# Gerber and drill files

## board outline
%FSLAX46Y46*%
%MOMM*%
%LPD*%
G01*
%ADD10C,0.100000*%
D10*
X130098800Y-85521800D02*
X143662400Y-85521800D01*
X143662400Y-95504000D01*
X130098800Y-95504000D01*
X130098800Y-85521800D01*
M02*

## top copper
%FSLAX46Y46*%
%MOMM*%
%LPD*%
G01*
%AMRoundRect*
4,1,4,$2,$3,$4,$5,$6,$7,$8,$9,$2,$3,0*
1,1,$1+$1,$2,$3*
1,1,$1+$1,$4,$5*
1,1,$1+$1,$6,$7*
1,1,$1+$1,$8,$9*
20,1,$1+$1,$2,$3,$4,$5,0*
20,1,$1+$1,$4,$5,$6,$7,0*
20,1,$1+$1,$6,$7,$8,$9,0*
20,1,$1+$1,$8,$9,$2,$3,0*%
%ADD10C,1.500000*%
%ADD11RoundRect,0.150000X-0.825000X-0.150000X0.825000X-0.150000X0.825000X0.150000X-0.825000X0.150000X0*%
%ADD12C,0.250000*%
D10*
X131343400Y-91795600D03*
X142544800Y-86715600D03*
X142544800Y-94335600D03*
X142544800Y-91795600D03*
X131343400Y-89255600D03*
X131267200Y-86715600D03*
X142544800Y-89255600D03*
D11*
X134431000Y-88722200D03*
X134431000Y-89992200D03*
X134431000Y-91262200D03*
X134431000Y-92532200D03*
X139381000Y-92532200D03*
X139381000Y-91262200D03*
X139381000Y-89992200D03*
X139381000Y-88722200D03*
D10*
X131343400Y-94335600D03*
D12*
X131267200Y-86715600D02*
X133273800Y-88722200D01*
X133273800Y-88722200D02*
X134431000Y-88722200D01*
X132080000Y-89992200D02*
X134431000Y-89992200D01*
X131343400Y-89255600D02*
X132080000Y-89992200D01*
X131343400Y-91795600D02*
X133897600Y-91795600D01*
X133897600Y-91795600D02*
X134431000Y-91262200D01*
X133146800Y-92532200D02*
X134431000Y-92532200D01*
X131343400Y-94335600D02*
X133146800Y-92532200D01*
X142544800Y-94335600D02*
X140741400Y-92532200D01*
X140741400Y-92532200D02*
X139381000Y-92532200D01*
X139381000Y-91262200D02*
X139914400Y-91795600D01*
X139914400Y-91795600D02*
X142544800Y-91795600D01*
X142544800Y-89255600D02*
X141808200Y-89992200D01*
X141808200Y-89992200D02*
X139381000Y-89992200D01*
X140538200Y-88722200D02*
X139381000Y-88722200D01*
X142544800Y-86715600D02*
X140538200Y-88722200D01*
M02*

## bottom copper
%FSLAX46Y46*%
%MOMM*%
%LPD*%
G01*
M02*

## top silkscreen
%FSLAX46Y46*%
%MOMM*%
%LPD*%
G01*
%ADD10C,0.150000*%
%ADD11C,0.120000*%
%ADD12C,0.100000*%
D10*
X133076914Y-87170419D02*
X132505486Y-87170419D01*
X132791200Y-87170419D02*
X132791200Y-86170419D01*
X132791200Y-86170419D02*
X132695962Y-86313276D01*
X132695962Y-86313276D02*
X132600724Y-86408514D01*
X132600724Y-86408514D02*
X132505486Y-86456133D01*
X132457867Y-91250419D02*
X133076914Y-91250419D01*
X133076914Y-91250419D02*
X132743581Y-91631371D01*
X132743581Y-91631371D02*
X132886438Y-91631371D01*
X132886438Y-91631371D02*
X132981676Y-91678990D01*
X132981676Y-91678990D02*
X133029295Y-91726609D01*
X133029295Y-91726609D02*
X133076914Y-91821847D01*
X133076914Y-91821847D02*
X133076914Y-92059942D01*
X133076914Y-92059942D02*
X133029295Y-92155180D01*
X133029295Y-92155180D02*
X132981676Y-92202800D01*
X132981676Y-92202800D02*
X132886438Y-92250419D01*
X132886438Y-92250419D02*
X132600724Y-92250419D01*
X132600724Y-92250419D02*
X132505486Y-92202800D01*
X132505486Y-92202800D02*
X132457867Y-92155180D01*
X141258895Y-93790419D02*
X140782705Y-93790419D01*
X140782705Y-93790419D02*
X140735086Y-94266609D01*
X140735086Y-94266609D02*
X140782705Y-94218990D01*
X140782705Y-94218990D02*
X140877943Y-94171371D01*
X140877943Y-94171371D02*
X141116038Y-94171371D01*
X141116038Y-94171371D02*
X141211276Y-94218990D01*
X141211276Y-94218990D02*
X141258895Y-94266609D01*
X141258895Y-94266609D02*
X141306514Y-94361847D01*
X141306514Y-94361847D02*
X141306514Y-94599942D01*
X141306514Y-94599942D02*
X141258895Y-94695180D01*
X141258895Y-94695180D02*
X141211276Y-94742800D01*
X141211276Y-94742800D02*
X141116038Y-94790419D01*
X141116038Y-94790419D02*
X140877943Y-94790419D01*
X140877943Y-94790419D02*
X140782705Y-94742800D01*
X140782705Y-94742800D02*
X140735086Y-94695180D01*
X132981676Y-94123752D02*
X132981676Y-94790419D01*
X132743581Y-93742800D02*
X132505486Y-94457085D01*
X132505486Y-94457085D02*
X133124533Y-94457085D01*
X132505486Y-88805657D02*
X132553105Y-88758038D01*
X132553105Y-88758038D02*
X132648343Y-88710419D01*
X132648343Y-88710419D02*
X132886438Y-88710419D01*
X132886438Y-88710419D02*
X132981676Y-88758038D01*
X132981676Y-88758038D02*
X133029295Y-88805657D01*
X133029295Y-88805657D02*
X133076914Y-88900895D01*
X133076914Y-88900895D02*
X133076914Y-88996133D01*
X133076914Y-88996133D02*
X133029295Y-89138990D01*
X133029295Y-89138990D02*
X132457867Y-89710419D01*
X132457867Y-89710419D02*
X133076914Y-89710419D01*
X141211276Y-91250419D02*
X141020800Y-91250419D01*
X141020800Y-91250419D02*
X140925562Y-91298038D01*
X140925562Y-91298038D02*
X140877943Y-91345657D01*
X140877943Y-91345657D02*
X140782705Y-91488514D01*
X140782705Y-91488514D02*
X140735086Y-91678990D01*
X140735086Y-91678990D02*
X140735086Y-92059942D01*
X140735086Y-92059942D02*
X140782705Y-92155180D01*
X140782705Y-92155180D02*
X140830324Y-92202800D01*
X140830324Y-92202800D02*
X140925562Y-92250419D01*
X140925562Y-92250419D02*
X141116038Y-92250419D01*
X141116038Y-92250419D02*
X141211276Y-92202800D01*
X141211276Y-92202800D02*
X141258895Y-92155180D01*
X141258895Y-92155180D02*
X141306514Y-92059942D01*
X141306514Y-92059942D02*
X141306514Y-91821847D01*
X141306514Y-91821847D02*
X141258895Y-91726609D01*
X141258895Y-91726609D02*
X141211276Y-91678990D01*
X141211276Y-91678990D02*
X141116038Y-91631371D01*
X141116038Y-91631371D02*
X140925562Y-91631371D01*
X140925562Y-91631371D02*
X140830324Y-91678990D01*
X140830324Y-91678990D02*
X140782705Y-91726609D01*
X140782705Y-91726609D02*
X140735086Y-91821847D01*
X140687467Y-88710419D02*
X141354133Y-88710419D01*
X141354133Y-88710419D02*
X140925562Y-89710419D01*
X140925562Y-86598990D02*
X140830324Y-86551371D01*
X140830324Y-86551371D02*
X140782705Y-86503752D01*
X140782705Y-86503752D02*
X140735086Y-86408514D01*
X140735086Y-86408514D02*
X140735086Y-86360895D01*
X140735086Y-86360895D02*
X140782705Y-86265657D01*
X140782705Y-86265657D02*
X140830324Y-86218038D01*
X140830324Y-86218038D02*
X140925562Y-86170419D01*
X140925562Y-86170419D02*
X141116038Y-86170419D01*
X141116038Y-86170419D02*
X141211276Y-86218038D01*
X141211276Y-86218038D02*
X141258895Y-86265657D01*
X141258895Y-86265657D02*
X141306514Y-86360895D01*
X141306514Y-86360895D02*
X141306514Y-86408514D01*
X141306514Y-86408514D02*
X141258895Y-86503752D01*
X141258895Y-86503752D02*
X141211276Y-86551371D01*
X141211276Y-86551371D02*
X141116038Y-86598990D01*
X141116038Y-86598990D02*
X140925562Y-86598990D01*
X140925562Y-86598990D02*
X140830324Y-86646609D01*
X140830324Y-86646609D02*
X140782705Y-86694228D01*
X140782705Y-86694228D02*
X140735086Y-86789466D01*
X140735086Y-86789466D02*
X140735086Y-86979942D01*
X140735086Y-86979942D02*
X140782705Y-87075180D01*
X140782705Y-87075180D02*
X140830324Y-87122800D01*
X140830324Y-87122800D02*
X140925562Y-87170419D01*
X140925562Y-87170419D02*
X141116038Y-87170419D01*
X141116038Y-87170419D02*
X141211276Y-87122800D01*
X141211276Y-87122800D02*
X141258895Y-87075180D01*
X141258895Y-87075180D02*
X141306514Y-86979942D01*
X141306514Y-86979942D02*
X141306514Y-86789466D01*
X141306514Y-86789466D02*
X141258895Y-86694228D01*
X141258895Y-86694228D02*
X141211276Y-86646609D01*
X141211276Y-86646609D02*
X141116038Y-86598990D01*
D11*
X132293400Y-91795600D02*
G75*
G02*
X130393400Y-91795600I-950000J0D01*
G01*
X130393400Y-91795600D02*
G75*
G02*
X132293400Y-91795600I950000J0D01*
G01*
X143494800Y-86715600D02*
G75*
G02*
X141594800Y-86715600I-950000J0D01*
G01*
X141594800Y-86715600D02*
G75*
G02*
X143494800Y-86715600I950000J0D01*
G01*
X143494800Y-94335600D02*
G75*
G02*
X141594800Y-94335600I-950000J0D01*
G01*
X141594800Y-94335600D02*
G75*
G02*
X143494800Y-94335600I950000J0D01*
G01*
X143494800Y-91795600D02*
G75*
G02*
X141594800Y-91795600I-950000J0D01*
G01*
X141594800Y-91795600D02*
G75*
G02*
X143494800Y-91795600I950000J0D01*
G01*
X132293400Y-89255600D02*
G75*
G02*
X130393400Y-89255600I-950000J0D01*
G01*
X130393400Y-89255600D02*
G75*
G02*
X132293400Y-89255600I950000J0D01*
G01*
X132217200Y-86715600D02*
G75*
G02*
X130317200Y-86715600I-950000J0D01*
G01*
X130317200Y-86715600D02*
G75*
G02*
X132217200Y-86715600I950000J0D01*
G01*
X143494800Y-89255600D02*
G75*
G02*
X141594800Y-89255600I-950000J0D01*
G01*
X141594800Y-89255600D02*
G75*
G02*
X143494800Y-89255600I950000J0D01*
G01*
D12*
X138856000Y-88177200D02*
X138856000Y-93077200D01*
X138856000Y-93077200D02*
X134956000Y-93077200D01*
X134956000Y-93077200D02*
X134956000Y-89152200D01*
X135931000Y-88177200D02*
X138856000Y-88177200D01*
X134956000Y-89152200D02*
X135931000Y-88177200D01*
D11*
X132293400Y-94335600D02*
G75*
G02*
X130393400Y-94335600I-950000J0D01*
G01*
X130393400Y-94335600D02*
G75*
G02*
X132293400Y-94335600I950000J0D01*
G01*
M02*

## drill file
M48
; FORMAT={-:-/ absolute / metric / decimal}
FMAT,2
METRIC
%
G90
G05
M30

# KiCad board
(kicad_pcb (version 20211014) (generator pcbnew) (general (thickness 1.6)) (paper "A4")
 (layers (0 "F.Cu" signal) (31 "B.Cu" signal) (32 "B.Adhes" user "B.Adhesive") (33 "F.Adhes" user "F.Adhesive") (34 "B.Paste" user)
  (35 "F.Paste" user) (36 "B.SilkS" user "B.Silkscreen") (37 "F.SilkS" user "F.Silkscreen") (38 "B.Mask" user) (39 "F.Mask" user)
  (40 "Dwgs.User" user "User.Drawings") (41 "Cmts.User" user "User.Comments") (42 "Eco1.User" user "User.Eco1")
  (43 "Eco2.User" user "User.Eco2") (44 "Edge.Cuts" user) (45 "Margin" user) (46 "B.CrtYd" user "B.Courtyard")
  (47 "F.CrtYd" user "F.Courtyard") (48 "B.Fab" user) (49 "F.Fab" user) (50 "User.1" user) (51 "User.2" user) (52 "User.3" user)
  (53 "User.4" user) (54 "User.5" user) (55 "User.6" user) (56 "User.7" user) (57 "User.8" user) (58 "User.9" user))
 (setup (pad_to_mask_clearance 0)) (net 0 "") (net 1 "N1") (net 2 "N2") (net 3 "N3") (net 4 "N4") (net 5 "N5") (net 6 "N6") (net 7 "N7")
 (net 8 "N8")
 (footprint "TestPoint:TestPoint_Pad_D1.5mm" (layer "F.Cu") (at 131.3434 91.7956)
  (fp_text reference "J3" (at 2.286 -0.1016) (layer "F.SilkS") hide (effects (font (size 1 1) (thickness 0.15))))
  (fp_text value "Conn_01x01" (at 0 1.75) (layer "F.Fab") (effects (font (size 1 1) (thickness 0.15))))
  (fp_circle (center 0 0) (end 0 0.95) (layer "F.SilkS") (width 0.12) (fill none))
  (pad "1" smd circle (at 0 0) (size 1.5 1.5) (layers "F.Cu" "F.Mask") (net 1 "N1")))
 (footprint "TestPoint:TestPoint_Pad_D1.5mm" (layer "F.Cu") (at 142.5448 86.7156)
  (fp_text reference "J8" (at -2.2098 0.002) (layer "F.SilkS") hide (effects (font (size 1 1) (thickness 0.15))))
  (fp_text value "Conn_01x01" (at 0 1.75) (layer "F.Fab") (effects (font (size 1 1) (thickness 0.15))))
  (fp_circle (center 0 0) (end 0 0.95) (layer "F.SilkS") (width 0.12) (fill none))
  (pad "1" smd circle (at 0 0) (size 1.5 1.5) (layers "F.Cu" "F.Mask") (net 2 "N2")))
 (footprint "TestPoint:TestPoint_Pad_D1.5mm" (layer "F.Cu") (at 142.5448 94.3356)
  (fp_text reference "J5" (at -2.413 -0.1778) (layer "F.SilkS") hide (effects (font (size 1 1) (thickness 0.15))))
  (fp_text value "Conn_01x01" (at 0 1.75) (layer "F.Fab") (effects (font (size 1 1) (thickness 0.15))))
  (fp_circle (center 0 0) (end 0 0.95) (layer "F.SilkS") (width 0.12) (fill none))
  (pad "1" smd circle (at 0 0) (size 1.5 1.5) (layers "F.Cu" "F.Mask") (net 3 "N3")))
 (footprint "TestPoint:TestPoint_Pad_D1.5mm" (layer "F.Cu") (at 142.5448 91.7956)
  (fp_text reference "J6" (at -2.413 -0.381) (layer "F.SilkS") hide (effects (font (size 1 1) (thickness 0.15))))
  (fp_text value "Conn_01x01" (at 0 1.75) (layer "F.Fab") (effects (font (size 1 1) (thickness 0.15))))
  (fp_circle (center 0 0) (end 0 0.95) (layer "F.SilkS") (width 0.12) (fill none))
  (pad "1" smd circle (at 0 0) (size 1.5 1.5) (layers "F.Cu" "F.Mask") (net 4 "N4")))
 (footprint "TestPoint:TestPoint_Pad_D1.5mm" (layer "F.Cu") (at 131.3434 89.2556)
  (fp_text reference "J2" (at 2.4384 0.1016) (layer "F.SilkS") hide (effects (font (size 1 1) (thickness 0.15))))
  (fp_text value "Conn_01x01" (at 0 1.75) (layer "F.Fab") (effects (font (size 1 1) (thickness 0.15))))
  (fp_circle (center 0 0) (end 0 0.95) (layer "F.SilkS") (width 0.12) (fill none))
  (pad "1" smd circle (at 0 0) (size 1.5 1.5) (layers "F.Cu" "F.Mask") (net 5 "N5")))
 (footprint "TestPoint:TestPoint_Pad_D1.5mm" (layer "F.Cu") (at 131.2672 86.7156)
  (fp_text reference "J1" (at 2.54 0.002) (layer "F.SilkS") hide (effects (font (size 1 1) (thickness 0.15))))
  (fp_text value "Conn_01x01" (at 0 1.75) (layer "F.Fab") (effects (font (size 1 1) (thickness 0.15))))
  (fp_circle (center 0 0) (end 0 0.95) (layer "F.SilkS") (width 0.12) (fill none))
  (pad "1" smd circle (at 0 0) (size 1.5 1.5) (layers "F.Cu" "F.Mask") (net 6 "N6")))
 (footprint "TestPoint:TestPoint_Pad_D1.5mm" (layer "F.Cu") (at 142.5448 89.2556)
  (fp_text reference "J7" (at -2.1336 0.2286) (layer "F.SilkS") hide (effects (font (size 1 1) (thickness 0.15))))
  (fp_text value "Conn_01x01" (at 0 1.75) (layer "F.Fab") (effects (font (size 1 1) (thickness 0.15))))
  (fp_circle (center 0 0) (end 0 0.95) (layer "F.SilkS") (width 0.12) (fill none))
  (pad "1" smd circle (at 0 0) (size 1.5 1.5) (layers "F.Cu" "F.Mask") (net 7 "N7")))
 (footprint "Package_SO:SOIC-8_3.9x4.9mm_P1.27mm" (layer "F.Cu") (at 136.906 90.6272)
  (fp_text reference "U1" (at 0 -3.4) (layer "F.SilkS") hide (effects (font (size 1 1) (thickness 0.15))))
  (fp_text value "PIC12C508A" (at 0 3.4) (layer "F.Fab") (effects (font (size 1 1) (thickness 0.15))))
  (fp_line (start 1.95 -2.45) (end 1.95 2.45) (layer "F.SilkS") (width 0.1))
  (fp_line (start 1.95 2.45) (end -1.95 2.45) (layer "F.SilkS") (width 0.1))
  (fp_line (start -1.95 2.45) (end -1.95 -1.475) (layer "F.SilkS") (width 0.1))
  (fp_line (start -0.975 -2.45) (end 1.95 -2.45) (layer "F.SilkS") (width 0.1))
  (fp_line (start -1.95 -1.475) (end -0.975 -2.45) (layer "F.SilkS") (width 0.1))
  (pad "1" smd roundrect (at -2.475 -1.905) (size 1.95 0.6) (layers "F.Cu" "F.Paste" "F.Mask") (roundrect_rratio 0.25) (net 6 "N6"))
  (pad "2" smd roundrect (at -2.475 -0.635) (size 1.95 0.6) (layers "F.Cu" "F.Paste" "F.Mask") (roundrect_rratio 0.25) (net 5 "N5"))
  (pad "3" smd roundrect (at -2.475 0.635) (size 1.95 0.6) (layers "F.Cu" "F.Paste" "F.Mask") (roundrect_rratio 0.25) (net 1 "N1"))
  (pad "4" smd roundrect (at -2.475 1.905) (size 1.95 0.6) (layers "F.Cu" "F.Paste" "F.Mask") (roundrect_rratio 0.25) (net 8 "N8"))
  (pad "5" smd roundrect (at 2.475 1.905) (size 1.95 0.6) (layers "F.Cu" "F.Paste" "F.Mask") (roundrect_rratio 0.25) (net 3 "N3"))
  (pad "6" smd roundrect (at 2.475 0.635) (size 1.95 0.6) (layers "F.Cu" "F.Paste" "F.Mask") (roundrect_rratio 0.25) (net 4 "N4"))
  (pad "7" smd roundrect (at 2.475 -0.635) (size 1.95 0.6) (layers "F.Cu" "F.Paste" "F.Mask") (roundrect_rratio 0.25) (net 7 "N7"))
  (pad "8" smd roundrect (at 2.475 -1.905) (size 1.95 0.6) (layers "F.Cu" "F.Paste" "F.Mask") (roundrect_rratio 0.25) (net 2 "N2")))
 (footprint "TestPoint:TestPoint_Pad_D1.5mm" (layer "F.Cu") (at 131.3434 94.3356)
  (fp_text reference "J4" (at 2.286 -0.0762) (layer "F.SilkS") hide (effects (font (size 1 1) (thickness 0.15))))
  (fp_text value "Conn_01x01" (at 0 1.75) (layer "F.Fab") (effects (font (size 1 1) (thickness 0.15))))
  (fp_circle (center 0 0) (end 0 0.95) (layer "F.SilkS") (width 0.12) (fill none))
  (pad "1" smd circle (at 0 0) (size 1.5 1.5) (layers "F.Cu" "F.Mask") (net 8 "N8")))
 (gr_rect (start 130.0988 85.5218) (end 143.6624 95.504) (layer "Edge.Cuts") (width 0.1) (fill none))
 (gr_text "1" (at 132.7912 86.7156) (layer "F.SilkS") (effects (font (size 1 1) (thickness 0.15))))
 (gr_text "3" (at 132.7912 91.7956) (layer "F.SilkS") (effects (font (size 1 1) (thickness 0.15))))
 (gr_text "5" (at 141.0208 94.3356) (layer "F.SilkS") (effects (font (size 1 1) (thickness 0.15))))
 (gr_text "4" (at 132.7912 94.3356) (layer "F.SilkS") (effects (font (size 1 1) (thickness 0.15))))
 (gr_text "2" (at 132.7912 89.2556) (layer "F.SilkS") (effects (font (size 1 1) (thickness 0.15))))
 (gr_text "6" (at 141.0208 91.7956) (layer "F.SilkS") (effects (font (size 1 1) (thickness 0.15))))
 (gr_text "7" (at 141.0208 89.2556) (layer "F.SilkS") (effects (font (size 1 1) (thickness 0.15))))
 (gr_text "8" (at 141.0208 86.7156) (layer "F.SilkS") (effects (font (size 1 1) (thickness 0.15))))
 (segment (start 131.2672 86.7156) (end 133.2738 88.7222) (width 0.25) (layer "F.Cu") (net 6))
 (segment (start 133.2738 88.7222) (end 134.431 88.7222) (width 0.25) (layer "F.Cu") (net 6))
 (segment (start 132.08 89.9922) (end 134.431 89.9922) (width 0.25) (layer "F.Cu") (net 5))
 (segment (start 131.3434 89.2556) (end 132.08 89.9922) (width 0.25) (layer "F.Cu") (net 5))
 (segment (start 131.3434 91.7956) (end 133.8976 91.7956) (width 0.25) (layer "F.Cu") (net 1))
 (segment (start 133.8976 91.7956) (end 134.431 91.2622) (width 0.25) (layer "F.Cu") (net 1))
 (segment (start 133.1468 92.5322) (end 134.431 92.5322) (width 0.25) (layer "F.Cu") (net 8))
 (segment (start 131.3434 94.3356) (end 133.1468 92.5322) (width 0.25) (layer "F.Cu") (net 8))
 (segment (start 142.5448 94.3356) (end 140.7414 92.5322) (width 0.25) (layer "F.Cu") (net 3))
 (segment (start 140.7414 92.5322) (end 139.381 92.5322) (width 0.25) (layer "F.Cu") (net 3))
 (segment (start 139.381 91.2622) (end 139.9144 91.7956) (width 0.25) (layer "F.Cu") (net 4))
 (segment (start 139.9144 91.7956) (end 142.5448 91.7956) (width 0.25) (layer "F.Cu") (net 4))
 (segment (start 142.5448 89.2556) (end 141.8082 89.9922) (width 0.25) (layer "F.Cu") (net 7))
 (segment (start 141.8082 89.9922) (end 139.381 89.9922) (width 0.25) (layer "F.Cu") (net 7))
 (segment (start 140.5382 88.7222) (end 139.381 88.7222) (width 0.25) (layer "F.Cu") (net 2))
 (segment (start 142.5448 86.7156) (end 140.5382 88.7222) (width 0.25) (layer "F.Cu") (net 2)))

